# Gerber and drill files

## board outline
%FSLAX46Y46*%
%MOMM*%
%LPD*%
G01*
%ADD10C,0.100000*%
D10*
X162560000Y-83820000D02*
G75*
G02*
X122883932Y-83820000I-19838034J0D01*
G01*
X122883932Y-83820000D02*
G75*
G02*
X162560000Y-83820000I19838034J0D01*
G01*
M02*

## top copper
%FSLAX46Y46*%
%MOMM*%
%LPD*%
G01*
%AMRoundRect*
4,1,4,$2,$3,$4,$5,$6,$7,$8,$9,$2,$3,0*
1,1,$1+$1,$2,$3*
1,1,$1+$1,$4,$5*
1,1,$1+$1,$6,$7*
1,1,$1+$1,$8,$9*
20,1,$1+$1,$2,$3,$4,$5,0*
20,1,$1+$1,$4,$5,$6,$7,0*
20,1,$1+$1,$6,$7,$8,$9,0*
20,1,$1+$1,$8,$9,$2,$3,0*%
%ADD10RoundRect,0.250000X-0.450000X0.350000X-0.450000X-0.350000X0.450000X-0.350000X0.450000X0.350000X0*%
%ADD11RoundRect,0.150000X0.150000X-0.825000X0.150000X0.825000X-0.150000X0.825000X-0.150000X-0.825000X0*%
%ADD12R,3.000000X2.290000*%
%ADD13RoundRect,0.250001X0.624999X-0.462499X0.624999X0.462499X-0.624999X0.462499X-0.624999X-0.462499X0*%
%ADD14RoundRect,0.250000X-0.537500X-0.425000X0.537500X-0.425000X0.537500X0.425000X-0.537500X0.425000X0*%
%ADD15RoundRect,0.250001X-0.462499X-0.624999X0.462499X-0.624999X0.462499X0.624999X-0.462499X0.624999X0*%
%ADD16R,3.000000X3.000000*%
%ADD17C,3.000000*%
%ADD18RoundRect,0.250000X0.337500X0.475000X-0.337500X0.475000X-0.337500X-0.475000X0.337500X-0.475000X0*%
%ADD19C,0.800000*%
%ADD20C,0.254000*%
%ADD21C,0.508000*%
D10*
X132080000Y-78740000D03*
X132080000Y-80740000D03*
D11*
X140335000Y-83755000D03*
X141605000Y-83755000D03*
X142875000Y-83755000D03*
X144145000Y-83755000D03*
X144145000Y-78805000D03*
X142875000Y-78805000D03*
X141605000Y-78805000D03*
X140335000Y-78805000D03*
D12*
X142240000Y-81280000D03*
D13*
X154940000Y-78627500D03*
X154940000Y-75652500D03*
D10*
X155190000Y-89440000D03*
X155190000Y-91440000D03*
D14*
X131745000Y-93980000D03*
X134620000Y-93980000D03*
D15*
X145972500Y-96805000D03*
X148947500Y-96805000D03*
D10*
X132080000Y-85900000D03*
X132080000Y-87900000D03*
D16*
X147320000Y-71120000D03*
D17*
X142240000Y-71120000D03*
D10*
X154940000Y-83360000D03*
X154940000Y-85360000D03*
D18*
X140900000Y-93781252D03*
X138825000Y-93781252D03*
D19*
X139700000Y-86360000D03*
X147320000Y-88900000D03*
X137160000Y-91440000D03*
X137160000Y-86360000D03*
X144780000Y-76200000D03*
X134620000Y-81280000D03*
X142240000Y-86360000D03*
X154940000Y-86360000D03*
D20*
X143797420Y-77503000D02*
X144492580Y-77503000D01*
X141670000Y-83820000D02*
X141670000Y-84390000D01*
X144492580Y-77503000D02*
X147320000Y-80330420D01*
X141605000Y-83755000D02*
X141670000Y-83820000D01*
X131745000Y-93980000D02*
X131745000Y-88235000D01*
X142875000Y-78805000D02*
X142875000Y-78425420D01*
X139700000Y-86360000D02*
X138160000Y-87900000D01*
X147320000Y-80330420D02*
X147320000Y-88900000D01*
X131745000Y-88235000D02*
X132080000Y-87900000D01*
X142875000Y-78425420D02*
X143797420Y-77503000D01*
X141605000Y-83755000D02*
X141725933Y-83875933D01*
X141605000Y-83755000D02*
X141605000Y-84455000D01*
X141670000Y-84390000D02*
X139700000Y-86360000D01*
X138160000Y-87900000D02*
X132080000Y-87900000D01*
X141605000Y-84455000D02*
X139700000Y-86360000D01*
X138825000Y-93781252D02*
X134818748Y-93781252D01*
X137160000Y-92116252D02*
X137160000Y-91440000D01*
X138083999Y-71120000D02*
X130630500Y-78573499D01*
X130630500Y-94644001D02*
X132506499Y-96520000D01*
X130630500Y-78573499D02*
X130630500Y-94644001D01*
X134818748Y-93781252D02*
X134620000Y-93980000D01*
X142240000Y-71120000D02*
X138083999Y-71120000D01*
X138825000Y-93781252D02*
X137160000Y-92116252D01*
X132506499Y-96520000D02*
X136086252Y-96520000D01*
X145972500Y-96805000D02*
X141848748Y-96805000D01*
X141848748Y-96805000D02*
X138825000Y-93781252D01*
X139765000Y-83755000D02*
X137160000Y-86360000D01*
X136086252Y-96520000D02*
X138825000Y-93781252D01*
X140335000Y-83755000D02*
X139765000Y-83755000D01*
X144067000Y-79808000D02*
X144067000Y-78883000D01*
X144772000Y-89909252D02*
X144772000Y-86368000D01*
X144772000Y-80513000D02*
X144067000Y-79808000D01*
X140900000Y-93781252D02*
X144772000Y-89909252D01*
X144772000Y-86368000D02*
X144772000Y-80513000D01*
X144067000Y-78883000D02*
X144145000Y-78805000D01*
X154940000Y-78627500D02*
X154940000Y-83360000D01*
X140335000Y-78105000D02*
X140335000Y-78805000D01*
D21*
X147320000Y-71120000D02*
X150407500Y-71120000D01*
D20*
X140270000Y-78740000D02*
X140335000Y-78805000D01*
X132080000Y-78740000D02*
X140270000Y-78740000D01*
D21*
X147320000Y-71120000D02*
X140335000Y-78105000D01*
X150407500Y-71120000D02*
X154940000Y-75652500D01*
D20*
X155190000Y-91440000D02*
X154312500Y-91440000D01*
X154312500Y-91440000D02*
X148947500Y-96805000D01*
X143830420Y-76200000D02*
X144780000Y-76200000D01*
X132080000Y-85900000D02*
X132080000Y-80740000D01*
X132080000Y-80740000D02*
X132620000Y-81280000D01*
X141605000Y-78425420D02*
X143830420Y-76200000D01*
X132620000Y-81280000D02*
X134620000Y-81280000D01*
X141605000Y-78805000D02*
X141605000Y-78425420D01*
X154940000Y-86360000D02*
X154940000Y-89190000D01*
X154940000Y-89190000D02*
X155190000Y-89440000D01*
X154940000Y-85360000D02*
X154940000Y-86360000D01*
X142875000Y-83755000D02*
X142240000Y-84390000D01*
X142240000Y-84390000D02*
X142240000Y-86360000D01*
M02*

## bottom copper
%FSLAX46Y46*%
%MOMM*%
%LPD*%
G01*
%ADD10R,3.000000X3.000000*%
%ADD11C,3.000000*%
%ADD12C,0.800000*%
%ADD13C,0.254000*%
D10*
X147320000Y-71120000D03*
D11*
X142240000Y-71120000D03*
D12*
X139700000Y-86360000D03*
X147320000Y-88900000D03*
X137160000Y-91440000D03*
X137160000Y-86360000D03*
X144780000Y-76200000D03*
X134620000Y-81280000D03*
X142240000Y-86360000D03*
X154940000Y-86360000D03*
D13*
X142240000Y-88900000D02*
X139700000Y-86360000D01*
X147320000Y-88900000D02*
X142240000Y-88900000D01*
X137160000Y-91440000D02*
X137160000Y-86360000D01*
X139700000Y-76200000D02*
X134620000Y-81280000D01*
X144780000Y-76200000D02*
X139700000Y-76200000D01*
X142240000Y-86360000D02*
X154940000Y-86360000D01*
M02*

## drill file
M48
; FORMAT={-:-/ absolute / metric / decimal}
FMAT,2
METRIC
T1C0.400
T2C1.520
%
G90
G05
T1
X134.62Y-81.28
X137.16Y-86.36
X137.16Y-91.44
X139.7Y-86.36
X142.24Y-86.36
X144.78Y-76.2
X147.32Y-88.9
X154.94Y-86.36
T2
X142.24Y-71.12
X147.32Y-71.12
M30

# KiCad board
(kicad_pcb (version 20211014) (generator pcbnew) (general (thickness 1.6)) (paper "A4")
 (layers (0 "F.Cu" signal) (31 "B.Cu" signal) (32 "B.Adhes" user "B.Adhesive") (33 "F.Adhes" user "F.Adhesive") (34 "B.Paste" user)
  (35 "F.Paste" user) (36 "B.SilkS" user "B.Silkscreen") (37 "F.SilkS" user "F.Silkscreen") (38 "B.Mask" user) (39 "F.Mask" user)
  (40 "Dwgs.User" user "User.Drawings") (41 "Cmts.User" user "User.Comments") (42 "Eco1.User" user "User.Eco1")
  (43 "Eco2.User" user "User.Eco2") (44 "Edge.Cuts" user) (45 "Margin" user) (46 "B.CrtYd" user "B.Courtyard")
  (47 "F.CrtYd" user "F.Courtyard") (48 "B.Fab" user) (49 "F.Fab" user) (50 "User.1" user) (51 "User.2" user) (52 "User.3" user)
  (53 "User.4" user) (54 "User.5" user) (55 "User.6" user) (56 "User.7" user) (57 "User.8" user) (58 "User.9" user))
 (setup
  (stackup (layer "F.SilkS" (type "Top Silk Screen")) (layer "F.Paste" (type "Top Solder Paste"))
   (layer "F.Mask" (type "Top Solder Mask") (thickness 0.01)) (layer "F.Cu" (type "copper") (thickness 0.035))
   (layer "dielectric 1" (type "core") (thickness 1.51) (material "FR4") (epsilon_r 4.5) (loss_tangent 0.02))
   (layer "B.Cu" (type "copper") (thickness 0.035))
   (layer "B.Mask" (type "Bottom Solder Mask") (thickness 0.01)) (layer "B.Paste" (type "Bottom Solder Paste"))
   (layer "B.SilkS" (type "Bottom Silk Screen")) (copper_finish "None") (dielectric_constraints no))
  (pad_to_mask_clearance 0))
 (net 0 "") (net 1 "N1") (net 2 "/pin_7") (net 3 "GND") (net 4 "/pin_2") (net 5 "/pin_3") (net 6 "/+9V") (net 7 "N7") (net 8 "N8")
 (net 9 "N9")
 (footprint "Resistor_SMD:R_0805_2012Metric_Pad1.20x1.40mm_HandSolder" (layer "F.Cu") (at 132.08 79.74 -90)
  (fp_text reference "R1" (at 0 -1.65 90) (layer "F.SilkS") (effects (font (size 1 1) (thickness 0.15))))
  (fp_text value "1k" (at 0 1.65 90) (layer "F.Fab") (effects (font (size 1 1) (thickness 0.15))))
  (pad "1" smd roundrect (at -1 0 270) (size 1.2 1.4) (layers "F.Cu" "F.Paste" "F.Mask") (roundrect_rratio 0.208333) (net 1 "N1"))
  (pad "2" smd roundrect (at 1 0 270) (size 1.2 1.4) (layers "F.Cu" "F.Paste" "F.Mask") (roundrect_rratio 0.208333) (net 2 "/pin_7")))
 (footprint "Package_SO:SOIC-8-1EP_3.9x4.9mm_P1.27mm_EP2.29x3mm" (layer "F.Cu") (at 142.24 81.28 90)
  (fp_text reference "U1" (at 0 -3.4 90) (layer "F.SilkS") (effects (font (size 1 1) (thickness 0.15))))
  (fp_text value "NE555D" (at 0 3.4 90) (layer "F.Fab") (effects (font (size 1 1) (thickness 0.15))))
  (pad "" smd roundrect (at 0.57 0.75 90) (size 0.92 1.21) (layers "F.Paste") (roundrect_rratio 0.25))
  (pad "" smd roundrect (at -0.57 -0.75 90) (size 0.92 1.21) (layers "F.Paste") (roundrect_rratio 0.25))
  (pad "" smd roundrect (at 0.57 -0.75 90) (size 0.92 1.21) (layers "F.Paste") (roundrect_rratio 0.25))
  (pad "" smd roundrect (at -0.57 0.75 90) (size 0.92 1.21) (layers "F.Paste") (roundrect_rratio 0.25))
  (pad "1" smd roundrect (at -2.475 -1.905 90) (size 1.95 0.6) (layers "F.Cu" "F.Paste" "F.Mask") (roundrect_rratio 0.25) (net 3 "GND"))
  (pad "2" smd roundrect (at -2.475 -0.635 90) (size 1.95 0.6) (layers "F.Cu" "F.Paste" "F.Mask") (roundrect_rratio 0.25) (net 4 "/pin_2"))
  (pad "3" smd roundrect (at -2.475 0.635 90) (size 1.95 0.6) (layers "F.Cu" "F.Paste" "F.Mask") (roundrect_rratio 0.25) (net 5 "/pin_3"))
  (pad "4" smd roundrect (at -2.475 1.905 90) (size 1.95 0.6) (layers "F.Cu" "F.Paste" "F.Mask") (roundrect_rratio 0.25) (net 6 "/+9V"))
  (pad "5" smd roundrect (at 2.475 1.905 90) (size 1.95 0.6) (layers "F.Cu" "F.Paste" "F.Mask") (roundrect_rratio 0.25) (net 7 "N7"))
  (pad "6" smd roundrect (at 2.475 0.635 90) (size 1.95 0.6) (layers "F.Cu" "F.Paste" "F.Mask") (roundrect_rratio 0.25) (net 4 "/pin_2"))
  (pad "7" smd roundrect (at 2.475 -0.635 90) (size 1.95 0.6) (layers "F.Cu" "F.Paste" "F.Mask") (roundrect_rratio 0.25) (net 2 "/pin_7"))
  (pad "8" smd roundrect (at 2.475 -1.905 90) (size 1.95 0.6) (layers "F.Cu" "F.Paste" "F.Mask") (roundrect_rratio 0.25) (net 1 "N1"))
  (pad "9" smd rect (at 0 0 90) (size 2.29 3) (layers "F.Cu" "F.Mask")))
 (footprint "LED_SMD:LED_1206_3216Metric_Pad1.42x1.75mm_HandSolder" (layer "F.Cu") (at 154.94 77.14 90)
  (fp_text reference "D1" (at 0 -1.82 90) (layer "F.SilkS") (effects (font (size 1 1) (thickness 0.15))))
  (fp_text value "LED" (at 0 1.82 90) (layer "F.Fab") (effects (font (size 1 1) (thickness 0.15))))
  (pad "1" smd roundrect (at -1.4875 0 90) (size 1.425 1.75) (layers "F.Cu" "F.Paste" "F.Mask") (roundrect_rratio 0.175439) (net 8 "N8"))
  (pad "2" smd roundrect (at 1.4875 0 90) (size 1.425 1.75) (layers "F.Cu" "F.Paste" "F.Mask") (roundrect_rratio 0.175439) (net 1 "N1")))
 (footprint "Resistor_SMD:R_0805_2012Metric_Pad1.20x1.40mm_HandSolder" (layer "F.Cu") (at 155.19 90.44 -90)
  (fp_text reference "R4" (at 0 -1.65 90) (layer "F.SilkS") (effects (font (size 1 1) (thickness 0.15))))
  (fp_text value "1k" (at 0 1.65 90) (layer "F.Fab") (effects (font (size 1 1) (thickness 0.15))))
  (pad "1" smd roundrect (at -1 0 270) (size 1.2 1.4) (layers "F.Cu" "F.Paste" "F.Mask") (roundrect_rratio 0.208333) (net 5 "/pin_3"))
  (pad "2" smd roundrect (at 1 0 270) (size 1.2 1.4) (layers "F.Cu" "F.Paste" "F.Mask") (roundrect_rratio 0.208333) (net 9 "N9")))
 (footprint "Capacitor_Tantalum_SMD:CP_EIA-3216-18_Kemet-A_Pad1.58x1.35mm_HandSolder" (layer "F.Cu") (at 133.1825 93.98)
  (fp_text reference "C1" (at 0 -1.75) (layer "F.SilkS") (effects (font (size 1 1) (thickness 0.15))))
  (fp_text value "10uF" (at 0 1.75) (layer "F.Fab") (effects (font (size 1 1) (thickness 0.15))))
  (pad "1" smd roundrect (at -1.4375 0) (size 1.575 1.35) (layers "F.Cu" "F.Paste" "F.Mask") (roundrect_rratio 0.185185) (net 4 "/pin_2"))
  (pad "2" smd roundrect (at 1.4375 0) (size 1.575 1.35) (layers "F.Cu" "F.Paste" "F.Mask") (roundrect_rratio 0.185185) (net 3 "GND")))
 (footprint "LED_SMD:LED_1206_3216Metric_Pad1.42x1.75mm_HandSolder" (layer "F.Cu") (at 147.46 96.805)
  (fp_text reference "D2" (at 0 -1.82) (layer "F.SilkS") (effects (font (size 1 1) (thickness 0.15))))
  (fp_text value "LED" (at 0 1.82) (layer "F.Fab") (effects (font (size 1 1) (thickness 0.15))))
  (pad "1" smd roundrect (at -1.4875 0) (size 1.425 1.75) (layers "F.Cu" "F.Paste" "F.Mask") (roundrect_rratio 0.175439) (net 3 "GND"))
  (pad "2" smd roundrect (at 1.4875 0) (size 1.425 1.75) (layers "F.Cu" "F.Paste" "F.Mask") (roundrect_rratio 0.175439) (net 9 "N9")))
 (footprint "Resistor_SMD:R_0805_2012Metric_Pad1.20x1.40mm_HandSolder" (layer "F.Cu") (at 132.08 86.9 -90)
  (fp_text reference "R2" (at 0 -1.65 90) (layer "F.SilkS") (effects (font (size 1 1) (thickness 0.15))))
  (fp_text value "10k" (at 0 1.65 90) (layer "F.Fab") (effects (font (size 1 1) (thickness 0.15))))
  (pad "1" smd roundrect (at -1 0 270) (size 1.2 1.4) (layers "F.Cu" "F.Paste" "F.Mask") (roundrect_rratio 0.208333) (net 2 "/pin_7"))
  (pad "2" smd roundrect (at 1 0 270) (size 1.2 1.4) (layers "F.Cu" "F.Paste" "F.Mask") (roundrect_rratio 0.208333) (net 4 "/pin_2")))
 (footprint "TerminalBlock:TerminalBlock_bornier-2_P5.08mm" (layer "F.Cu") (at 147.32 71.12 180)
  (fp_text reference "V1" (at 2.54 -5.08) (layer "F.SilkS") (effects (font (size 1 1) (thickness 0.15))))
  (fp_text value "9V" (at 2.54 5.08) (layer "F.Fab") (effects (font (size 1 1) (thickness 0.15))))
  (pad "1" thru_hole rect (at 0 0 180) (size 3 3) (drill 1.52) (layers *.Cu *.Mask) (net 1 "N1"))
  (pad "2" thru_hole circle (at 5.08 0 180) (size 3 3) (drill 1.52) (layers *.Cu *.Mask) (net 3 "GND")))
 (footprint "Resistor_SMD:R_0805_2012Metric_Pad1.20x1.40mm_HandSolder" (layer "F.Cu") (at 154.94 84.36 -90)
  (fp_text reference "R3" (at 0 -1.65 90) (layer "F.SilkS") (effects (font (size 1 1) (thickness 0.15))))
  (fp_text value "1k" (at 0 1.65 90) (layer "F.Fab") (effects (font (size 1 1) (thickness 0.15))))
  (pad "1" smd roundrect (at -1 0 270) (size 1.2 1.4) (layers "F.Cu" "F.Paste" "F.Mask") (roundrect_rratio 0.208333) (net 8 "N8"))
  (pad "2" smd roundrect (at 1 0 270) (size 1.2 1.4) (layers "F.Cu" "F.Paste" "F.Mask") (roundrect_rratio 0.208333) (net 5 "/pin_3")))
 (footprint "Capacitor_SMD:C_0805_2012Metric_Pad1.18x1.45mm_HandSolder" (layer "F.Cu") (at 139.8625 93.781252 180)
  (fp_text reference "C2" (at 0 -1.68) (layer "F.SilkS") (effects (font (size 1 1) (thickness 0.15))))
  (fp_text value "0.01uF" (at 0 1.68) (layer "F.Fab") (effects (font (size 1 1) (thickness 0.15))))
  (pad "1" smd roundrect (at -1.0375 0 180) (size 1.175 1.45) (layers "F.Cu" "F.Paste" "F.Mask") (roundrect_rratio 0.212766) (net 7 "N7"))
  (pad "2" smd roundrect (at 1.0375 0 180) (size 1.175 1.45) (layers "F.Cu" "F.Paste" "F.Mask") (roundrect_rratio 0.212766) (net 3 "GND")))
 (gr_circle (center 142.721966 83.82) (end 157.961966 96.52) (layer "Edge.Cuts") (width 0.1) (fill none))
 (segment (start 143.79742 77.503) (end 144.49258 77.503) (width 0.254) (layer "F.Cu") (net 4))
 (segment (start 141.67 83.82) (end 141.67 84.39) (width 0.254) (layer "F.Cu") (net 4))
 (segment (start 144.49258 77.503) (end 147.32 80.33042) (width 0.254) (layer "F.Cu") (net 4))
 (segment (start 141.605 83.755) (end 141.67 83.82) (width 0.254) (layer "F.Cu") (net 4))
 (segment (start 131.745 93.98) (end 131.745 88.235) (width 0.254) (layer "F.Cu") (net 4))
 (segment (start 142.875 78.805) (end 142.875 78.42542) (width 0.254) (layer "F.Cu") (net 4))
 (segment (start 139.7 86.36) (end 138.16 87.9) (width 0.254) (layer "F.Cu") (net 4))
 (segment (start 147.32 80.33042) (end 147.32 88.9) (width 0.254) (layer "F.Cu") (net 4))
 (segment (start 131.745 88.235) (end 132.08 87.9) (width 0.254) (layer "F.Cu") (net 4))
 (segment (start 142.875 78.42542) (end 143.79742 77.503) (width 0.254) (layer "F.Cu") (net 4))
 (segment (start 141.605 83.755) (end 141.725933 83.875933) (width 0.254) (layer "F.Cu") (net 4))
 (segment (start 141.605 83.755) (end 141.605 84.455) (width 0.254) (layer "F.Cu") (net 4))
 (segment (start 141.67 84.39) (end 139.7 86.36) (width 0.254) (layer "F.Cu") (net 4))
 (segment (start 138.16 87.9) (end 132.08 87.9) (width 0.254) (layer "F.Cu") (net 4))
 (segment (start 141.605 84.455) (end 139.7 86.36) (width 0.254) (layer "F.Cu") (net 4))
 (via (at 139.7 86.36) (size 0.8) (drill 0.4) (layers "F.Cu" "B.Cu") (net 4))
 (via (at 147.32 88.9) (size 0.8) (drill 0.4) (layers "F.Cu" "B.Cu") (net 4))
 (segment (start 142.24 88.9) (end 139.7 86.36) (width 0.254) (layer "B.Cu") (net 4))
 (segment (start 147.32 88.9) (end 142.24 88.9) (width 0.254) (layer "B.Cu") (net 4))
 (segment (start 138.825 93.781252) (end 134.818748 93.781252) (width 0.254) (layer "F.Cu") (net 3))
 (segment (start 137.16 92.116252) (end 137.16 91.44) (width 0.254) (layer "F.Cu") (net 3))
 (segment (start 138.083999 71.12) (end 130.6305 78.573499) (width 0.254) (layer "F.Cu") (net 3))
 (segment (start 130.6305 94.644001) (end 132.506499 96.52) (width 0.254) (layer "F.Cu") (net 3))
 (segment (start 130.6305 78.573499) (end 130.6305 94.644001) (width 0.254) (layer "F.Cu") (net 3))
 (segment (start 134.818748 93.781252) (end 134.62 93.98) (width 0.254) (layer "F.Cu") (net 3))
 (segment (start 142.24 71.12) (end 138.083999 71.12) (width 0.254) (layer "F.Cu") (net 3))
 (segment (start 138.825 93.781252) (end 137.16 92.116252) (width 0.254) (layer "F.Cu") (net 3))
 (segment (start 132.506499 96.52) (end 136.086252 96.52) (width 0.254) (layer "F.Cu") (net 3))
 (segment (start 145.9725 96.805) (end 141.848748 96.805) (width 0.254) (layer "F.Cu") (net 3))
 (segment (start 141.848748 96.805) (end 138.825 93.781252) (width 0.254) (layer "F.Cu") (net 3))
 (segment (start 139.765 83.755) (end 137.16 86.36) (width 0.254) (layer "F.Cu") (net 3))
 (segment (start 136.086252 96.52) (end 138.825 93.781252) (width 0.254) (layer "F.Cu") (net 3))
 (segment (start 140.335 83.755) (end 139.765 83.755) (width 0.254) (layer "F.Cu") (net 3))
 (via (at 137.16 91.44) (size 0.8) (drill 0.4) (layers "F.Cu" "B.Cu") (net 3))
 (via (at 137.16 86.36) (size 0.8) (drill 0.4) (layers "F.Cu" "B.Cu") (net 3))
 (segment (start 137.16 91.44) (end 137.16 86.36) (width 0.254) (layer "B.Cu") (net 3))
 (segment (start 144.067 79.808) (end 144.067 78.883) (width 0.254) (layer "F.Cu") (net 7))
 (segment (start 144.772 89.909252) (end 144.772 86.368) (width 0.254) (layer "F.Cu") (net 7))
 (segment (start 144.772 80.513) (end 144.067 79.808) (width 0.254) (layer "F.Cu") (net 7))
 (segment (start 140.9 93.781252) (end 144.772 89.909252) (width 0.254) (layer "F.Cu") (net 7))
 (segment (start 144.772 86.368) (end 144.772 80.513) (width 0.254) (layer "F.Cu") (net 7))
 (segment (start 144.067 78.883) (end 144.145 78.805) (width 0.254) (layer "F.Cu") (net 7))
 (segment (start 154.94 78.6275) (end 154.94 83.36) (width 0.254) (layer "F.Cu") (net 8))
 (segment (start 140.335 78.105) (end 140.335 78.805) (width 0.254) (layer "F.Cu") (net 1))
 (segment (start 147.32 71.12) (end 150.4075 71.12) (width 0.508) (layer "F.Cu") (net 1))
 (segment (start 140.27 78.74) (end 140.335 78.805) (width 0.254) (layer "F.Cu") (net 1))
 (segment (start 132.08 78.74) (end 140.27 78.74) (width 0.254) (layer "F.Cu") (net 1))
 (segment (start 147.32 71.12) (end 140.335 78.105) (width 0.508) (layer "F.Cu") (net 1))
 (segment (start 150.4075 71.12) (end 154.94 75.6525) (width 0.508) (layer "F.Cu") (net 1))
 (segment (start 155.19 91.44) (end 154.3125 91.44) (width 0.254) (layer "F.Cu") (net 9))
 (segment (start 154.3125 91.44) (end 148.9475 96.805) (width 0.254) (layer "F.Cu") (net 9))
 (segment (start 143.83042 76.2) (end 144.78 76.2) (width 0.254) (layer "F.Cu") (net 2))
 (segment (start 132.08 85.9) (end 132.08 80.74) (width 0.254) (layer "F.Cu") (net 2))
 (segment (start 132.08 80.74) (end 132.62 81.28) (width 0.254) (layer "F.Cu") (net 2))
 (segment (start 141.605 78.42542) (end 143.83042 76.2) (width 0.254) (layer "F.Cu") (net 2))
 (segment (start 132.62 81.28) (end 134.62 81.28) (width 0.254) (layer "F.Cu") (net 2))
 (segment (start 141.605 78.805) (end 141.605 78.42542) (width 0.254) (layer "F.Cu") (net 2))
 (via (at 144.78 76.2) (size 0.8) (drill 0.4) (layers "F.Cu" "B.Cu") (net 2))
 (via (at 134.62 81.28) (size 0.8) (drill 0.4) (layers "F.Cu" "B.Cu") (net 2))
 (segment (start 139.7 76.2) (end 134.62 81.28) (width 0.254) (layer "B.Cu") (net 2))
 (segment (start 144.78 76.2) (end 139.7 76.2) (width 0.254) (layer "B.Cu") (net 2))
 (segment (start 154.94 86.36) (end 154.94 89.19) (width 0.254) (layer "F.Cu") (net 5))
 (segment (start 154.94 89.19) (end 155.19 89.44) (width 0.254) (layer "F.Cu") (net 5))
 (segment (start 154.94 85.36) (end 154.94 86.36) (width 0.254) (layer "F.Cu") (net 5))
 (segment (start 142.875 83.755) (end 142.24 84.39) (width 0.254) (layer "F.Cu") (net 5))
 (segment (start 142.24 84.39) (end 142.24 86.36) (width 0.254) (layer "F.Cu") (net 5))
 (via (at 142.24 86.36) (size 0.8) (drill 0.4) (layers "F.Cu" "B.Cu") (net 5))
 (via (at 154.94 86.36) (size 0.8) (drill 0.4) (layers "F.Cu" "B.Cu") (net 5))
 (segment (start 142.24 86.36) (end 154.94 86.36) (width 0.254) (layer "B.Cu") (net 5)))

